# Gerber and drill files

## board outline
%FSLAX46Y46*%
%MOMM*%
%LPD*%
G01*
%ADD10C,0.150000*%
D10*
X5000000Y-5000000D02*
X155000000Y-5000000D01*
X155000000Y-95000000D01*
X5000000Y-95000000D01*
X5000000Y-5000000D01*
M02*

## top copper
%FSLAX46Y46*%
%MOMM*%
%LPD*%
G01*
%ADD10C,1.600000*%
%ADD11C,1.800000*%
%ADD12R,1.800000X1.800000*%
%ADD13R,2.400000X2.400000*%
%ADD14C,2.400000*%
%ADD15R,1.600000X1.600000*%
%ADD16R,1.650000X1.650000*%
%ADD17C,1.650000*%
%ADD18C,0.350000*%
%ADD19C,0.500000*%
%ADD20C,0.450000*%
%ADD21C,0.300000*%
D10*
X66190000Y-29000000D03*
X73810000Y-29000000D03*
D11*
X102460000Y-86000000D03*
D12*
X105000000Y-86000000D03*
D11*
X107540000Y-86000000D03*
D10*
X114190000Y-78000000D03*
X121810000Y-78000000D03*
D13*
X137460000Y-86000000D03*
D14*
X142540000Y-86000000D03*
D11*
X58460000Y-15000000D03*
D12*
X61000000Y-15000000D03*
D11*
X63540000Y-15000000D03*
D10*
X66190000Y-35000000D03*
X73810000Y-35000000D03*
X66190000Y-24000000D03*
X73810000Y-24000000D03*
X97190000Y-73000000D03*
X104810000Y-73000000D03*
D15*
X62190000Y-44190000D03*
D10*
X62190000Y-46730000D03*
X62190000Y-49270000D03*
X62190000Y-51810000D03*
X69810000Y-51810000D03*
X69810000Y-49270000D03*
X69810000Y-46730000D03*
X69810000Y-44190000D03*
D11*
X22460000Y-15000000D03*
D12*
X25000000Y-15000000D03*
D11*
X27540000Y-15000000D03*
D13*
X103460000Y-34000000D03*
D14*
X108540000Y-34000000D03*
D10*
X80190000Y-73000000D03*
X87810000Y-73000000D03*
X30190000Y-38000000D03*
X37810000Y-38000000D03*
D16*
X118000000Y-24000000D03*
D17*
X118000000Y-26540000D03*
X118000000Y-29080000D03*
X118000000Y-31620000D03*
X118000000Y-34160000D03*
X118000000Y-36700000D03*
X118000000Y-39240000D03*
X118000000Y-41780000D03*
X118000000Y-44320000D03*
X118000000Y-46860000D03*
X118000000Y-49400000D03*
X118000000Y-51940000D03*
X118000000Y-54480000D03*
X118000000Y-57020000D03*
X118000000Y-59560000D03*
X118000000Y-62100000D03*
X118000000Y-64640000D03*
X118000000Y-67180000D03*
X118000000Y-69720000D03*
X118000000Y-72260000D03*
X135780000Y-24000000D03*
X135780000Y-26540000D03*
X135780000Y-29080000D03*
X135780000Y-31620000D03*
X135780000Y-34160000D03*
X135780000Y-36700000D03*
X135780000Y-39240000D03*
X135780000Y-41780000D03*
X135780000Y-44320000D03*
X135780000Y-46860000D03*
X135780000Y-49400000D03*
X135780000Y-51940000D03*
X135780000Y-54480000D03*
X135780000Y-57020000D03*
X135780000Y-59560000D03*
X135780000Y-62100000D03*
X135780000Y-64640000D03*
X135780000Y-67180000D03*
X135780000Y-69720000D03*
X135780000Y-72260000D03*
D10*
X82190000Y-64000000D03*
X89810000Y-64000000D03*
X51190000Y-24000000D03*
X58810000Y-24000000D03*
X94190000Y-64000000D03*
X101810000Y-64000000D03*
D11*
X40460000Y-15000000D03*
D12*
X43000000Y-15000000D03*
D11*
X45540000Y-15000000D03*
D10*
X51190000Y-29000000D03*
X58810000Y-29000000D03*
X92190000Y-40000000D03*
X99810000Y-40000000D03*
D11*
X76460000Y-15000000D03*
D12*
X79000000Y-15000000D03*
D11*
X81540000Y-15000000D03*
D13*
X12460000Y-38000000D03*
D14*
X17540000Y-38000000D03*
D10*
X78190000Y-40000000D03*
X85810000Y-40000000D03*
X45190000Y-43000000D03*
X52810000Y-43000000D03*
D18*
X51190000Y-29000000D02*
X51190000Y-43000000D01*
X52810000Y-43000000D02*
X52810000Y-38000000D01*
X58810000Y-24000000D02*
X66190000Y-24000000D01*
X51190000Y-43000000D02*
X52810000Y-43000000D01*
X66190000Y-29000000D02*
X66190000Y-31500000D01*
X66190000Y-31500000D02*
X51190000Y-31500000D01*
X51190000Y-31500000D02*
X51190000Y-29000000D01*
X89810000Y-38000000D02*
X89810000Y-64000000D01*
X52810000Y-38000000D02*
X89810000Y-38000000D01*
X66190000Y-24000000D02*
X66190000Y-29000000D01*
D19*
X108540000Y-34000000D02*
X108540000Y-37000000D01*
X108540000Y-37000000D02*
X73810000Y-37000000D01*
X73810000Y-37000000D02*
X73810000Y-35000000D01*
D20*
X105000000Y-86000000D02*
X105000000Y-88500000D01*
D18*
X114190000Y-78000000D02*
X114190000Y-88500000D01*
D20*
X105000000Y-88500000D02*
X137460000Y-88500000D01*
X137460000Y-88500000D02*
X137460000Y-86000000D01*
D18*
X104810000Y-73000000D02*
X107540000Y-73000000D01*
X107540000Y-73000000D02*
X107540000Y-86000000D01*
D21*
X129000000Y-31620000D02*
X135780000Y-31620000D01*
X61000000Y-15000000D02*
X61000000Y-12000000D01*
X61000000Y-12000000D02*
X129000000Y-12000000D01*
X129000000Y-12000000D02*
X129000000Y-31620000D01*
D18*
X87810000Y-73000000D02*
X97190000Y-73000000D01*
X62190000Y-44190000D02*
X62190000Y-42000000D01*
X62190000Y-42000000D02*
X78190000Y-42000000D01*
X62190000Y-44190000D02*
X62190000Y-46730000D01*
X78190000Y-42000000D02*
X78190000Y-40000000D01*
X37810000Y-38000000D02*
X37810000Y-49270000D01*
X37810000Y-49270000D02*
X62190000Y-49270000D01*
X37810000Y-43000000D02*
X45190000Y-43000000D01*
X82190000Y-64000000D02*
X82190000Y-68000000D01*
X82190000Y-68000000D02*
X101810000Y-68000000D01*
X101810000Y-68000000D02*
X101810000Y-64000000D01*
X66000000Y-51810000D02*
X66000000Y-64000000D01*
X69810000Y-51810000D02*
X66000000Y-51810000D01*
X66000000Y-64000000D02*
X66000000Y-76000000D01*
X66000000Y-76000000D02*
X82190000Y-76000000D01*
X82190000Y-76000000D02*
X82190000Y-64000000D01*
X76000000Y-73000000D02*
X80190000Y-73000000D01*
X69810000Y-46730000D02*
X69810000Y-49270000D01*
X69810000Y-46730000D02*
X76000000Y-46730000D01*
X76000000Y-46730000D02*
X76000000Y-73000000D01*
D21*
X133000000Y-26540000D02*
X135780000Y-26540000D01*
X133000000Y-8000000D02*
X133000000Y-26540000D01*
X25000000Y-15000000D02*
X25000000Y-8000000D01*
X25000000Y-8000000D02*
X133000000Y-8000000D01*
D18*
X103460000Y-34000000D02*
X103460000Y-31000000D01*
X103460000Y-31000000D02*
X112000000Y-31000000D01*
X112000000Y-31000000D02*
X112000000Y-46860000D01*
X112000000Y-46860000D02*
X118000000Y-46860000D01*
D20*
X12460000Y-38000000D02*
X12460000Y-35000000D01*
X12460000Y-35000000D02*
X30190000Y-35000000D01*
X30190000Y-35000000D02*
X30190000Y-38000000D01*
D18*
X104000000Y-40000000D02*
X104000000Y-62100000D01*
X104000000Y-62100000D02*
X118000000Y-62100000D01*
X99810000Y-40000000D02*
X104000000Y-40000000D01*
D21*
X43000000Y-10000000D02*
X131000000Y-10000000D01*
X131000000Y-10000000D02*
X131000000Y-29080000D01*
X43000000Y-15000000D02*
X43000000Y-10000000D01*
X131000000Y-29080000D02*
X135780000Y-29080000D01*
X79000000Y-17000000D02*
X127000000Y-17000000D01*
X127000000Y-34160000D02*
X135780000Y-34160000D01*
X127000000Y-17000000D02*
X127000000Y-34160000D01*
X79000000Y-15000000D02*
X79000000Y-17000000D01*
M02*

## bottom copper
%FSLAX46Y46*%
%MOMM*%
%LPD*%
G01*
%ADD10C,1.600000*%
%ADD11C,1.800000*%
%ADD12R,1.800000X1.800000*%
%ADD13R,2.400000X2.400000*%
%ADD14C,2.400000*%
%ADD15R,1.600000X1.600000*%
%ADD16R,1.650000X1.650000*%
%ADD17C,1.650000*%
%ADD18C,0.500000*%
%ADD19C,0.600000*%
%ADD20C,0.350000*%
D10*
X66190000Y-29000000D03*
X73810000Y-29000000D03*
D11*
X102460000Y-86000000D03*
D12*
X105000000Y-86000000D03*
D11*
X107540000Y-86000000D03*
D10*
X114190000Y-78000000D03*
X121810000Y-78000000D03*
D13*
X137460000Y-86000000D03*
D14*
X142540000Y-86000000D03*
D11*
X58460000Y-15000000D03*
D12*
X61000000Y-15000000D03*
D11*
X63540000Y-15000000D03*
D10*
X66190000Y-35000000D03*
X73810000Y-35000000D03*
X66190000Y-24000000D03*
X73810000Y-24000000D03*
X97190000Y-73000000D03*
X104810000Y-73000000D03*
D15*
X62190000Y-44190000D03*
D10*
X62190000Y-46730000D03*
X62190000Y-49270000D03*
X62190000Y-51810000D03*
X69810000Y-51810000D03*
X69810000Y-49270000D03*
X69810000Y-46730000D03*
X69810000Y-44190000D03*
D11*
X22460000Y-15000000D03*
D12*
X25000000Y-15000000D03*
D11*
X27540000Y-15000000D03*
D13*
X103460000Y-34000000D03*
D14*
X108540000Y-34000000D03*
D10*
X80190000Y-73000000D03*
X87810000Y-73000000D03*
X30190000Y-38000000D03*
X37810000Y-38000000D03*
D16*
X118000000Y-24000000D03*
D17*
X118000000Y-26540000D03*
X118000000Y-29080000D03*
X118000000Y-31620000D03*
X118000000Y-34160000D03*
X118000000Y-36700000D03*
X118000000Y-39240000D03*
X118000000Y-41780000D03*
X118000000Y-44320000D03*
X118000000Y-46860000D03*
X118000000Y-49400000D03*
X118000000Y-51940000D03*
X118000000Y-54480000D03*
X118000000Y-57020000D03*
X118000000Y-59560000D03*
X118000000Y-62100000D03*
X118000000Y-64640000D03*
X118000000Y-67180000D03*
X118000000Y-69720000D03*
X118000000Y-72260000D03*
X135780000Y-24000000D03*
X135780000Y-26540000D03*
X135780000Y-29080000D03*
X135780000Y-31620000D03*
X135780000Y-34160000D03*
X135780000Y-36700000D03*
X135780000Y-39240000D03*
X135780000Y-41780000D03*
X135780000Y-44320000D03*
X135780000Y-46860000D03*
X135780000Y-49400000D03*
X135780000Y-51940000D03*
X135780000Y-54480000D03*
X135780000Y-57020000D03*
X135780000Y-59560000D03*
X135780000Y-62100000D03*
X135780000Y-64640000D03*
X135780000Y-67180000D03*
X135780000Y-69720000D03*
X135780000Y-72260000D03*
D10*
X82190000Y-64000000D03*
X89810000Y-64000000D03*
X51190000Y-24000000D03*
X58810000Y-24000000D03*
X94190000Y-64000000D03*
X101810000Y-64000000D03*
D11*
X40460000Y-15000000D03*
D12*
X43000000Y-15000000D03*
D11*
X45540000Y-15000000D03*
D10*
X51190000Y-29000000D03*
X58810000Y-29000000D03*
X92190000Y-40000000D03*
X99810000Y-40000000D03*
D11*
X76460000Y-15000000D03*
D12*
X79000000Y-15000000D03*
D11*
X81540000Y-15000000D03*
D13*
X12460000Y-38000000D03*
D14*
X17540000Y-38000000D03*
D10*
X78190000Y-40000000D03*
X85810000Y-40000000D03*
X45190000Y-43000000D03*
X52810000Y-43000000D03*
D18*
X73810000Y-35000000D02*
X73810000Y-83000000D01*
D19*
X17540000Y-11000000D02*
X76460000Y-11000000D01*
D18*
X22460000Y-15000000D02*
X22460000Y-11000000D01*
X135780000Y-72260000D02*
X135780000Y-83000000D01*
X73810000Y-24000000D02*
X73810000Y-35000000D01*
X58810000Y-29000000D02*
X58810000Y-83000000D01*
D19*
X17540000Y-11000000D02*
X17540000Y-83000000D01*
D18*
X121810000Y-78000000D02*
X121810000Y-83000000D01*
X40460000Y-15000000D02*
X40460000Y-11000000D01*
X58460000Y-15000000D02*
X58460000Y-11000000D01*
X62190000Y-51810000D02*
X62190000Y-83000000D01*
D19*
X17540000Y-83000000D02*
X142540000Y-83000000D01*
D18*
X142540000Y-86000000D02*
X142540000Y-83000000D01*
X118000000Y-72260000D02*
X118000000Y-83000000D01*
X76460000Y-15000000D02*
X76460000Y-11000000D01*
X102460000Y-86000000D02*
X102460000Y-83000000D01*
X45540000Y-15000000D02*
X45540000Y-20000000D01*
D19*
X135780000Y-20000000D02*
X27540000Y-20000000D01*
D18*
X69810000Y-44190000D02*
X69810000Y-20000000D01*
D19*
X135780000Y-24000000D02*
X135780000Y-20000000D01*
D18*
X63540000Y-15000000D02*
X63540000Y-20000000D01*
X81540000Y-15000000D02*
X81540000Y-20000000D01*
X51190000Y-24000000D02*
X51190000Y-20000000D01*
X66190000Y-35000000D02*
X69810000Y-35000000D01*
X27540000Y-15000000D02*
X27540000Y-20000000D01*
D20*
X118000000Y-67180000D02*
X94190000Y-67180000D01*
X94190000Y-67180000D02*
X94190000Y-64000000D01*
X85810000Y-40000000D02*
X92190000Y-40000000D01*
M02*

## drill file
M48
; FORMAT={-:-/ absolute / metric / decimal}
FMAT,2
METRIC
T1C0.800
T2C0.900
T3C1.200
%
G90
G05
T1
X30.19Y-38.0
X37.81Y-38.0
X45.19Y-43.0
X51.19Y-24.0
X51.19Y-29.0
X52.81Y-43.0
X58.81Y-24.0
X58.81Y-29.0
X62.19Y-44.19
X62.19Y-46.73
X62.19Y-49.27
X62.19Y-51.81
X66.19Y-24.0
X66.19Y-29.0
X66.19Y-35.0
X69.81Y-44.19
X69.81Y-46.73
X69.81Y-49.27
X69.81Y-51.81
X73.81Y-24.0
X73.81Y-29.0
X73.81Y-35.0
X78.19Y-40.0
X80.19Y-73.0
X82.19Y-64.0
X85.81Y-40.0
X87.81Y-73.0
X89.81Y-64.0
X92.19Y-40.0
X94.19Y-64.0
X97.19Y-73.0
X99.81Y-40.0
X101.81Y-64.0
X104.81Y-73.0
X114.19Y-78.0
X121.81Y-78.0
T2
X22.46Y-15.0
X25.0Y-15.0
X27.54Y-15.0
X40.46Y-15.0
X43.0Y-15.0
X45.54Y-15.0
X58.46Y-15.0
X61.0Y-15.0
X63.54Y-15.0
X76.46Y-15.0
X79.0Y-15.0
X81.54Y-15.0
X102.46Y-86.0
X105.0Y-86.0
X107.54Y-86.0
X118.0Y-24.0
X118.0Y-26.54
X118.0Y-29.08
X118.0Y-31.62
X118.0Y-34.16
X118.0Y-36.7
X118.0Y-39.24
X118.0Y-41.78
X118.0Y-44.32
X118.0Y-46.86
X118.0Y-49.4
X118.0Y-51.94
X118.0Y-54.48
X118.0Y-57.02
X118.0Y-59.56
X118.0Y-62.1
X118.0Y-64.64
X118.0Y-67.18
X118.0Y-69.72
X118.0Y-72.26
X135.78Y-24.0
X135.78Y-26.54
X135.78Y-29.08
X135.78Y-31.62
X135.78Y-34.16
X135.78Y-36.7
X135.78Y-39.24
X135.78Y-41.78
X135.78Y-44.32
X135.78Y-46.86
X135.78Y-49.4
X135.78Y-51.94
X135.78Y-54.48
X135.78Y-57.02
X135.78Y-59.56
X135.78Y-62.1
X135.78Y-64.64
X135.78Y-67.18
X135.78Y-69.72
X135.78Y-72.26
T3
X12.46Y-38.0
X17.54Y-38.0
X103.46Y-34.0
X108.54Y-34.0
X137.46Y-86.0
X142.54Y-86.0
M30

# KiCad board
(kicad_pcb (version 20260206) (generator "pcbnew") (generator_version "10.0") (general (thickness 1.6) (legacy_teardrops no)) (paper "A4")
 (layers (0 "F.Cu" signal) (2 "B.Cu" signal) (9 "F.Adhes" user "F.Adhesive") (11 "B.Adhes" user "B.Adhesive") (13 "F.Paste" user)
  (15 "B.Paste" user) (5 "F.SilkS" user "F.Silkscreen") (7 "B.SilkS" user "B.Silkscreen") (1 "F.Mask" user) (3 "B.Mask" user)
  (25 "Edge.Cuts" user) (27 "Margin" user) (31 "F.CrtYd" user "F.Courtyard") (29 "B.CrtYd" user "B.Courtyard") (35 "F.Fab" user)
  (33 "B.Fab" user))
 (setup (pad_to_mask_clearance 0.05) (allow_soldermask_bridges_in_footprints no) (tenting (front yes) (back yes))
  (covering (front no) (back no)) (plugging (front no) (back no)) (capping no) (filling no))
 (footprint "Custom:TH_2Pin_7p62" (layer "F.Cu") (at 70 29)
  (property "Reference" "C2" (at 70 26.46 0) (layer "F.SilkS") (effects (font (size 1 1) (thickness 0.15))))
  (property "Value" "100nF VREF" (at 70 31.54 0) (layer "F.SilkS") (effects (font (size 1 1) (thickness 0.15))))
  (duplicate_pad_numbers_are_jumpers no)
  (pad "1" thru_hole circle (at -3.81 0) (size 1.6 1.6) (drill 0.8) (layers "*.Cu" "*.Mask") (remove_unused_layers no) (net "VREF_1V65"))
  (pad "2" thru_hole circle (at 3.81 0) (size 1.6 1.6) (drill 0.8) (layers "*.Cu" "*.Mask") (remove_unused_layers no) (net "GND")))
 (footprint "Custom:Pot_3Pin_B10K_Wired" (layer "F.Cu") (at 105 86)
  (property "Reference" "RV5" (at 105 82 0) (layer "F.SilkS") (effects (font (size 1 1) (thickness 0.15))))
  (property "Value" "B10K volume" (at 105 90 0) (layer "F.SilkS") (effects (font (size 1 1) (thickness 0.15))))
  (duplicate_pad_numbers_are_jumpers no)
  (pad "1" thru_hole circle (at -2.54 0) (size 1.8 1.8) (drill 0.9) (layers "*.Cu" "*.Mask") (remove_unused_layers no) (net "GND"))
  (pad "2" thru_hole rect (at 0 0) (size 1.8 1.8) (drill 0.9) (layers "*.Cu" "*.Mask") (remove_unused_layers no) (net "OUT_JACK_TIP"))
  (pad "3" thru_hole circle (at 2.54 0) (size 1.8 1.8) (drill 0.9) (layers "*.Cu" "*.Mask") (remove_unused_layers no) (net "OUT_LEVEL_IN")))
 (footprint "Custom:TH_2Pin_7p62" (layer "F.Cu") (at 118 78)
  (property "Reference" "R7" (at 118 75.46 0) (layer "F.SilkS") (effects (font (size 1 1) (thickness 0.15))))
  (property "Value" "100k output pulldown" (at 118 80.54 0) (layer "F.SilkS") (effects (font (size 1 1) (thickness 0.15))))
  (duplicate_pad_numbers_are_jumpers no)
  (pad "1" thru_hole circle (at -3.81 0) (size 1.6 1.6) (drill 0.8) (layers "*.Cu" "*.Mask") (remove_unused_layers no) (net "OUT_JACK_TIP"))
  (pad "2" thru_hole circle (at 3.81 0) (size 1.6 1.6) (drill 0.8) (layers "*.Cu" "*.Mask") (remove_unused_layers no) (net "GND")))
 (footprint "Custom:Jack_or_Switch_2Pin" (layer "F.Cu") (at 140 86)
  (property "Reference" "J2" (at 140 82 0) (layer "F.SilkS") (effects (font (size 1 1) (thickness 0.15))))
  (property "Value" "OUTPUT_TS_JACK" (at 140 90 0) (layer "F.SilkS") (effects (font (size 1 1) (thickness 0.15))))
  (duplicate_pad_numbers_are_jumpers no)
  (pad "1" thru_hole rect (at -2.54 0) (size 2.4 2.4) (drill 1.2) (layers "*.Cu" "*.Mask") (remove_unused_layers no) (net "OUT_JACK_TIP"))
  (pad "2" thru_hole circle (at 2.54 0) (size 2.4 2.4) (drill 1.2) (layers "*.Cu" "*.Mask") (remove_unused_layers no) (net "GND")))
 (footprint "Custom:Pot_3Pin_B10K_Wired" (layer "F.Cu") (at 61 15)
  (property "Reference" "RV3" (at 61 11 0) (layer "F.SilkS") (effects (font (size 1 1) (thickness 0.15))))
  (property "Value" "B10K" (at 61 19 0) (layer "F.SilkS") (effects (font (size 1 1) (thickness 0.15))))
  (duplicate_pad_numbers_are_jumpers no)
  (pad "1" thru_hole circle (at -2.54 0) (size 1.8 1.8) (drill 0.9) (layers "*.Cu" "*.Mask") (remove_unused_layers no) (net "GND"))
  (pad "2" thru_hole rect (at 0 0) (size 1.8 1.8) (drill 0.9) (layers "*.Cu" "*.Mask") (remove_unused_layers no) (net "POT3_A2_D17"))
  (pad "3" thru_hole circle (at 2.54 0) (size 1.8 1.8) (drill 0.9) (layers "*.Cu" "*.Mask") (remove_unused_layers no) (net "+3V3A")))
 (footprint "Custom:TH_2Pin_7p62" (layer "F.Cu") (at 70 35)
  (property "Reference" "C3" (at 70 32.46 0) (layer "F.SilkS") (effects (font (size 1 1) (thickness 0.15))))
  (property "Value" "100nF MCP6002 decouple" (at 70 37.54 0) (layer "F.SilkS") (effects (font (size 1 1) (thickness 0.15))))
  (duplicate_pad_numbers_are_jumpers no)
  (pad "1" thru_hole circle (at -3.81 0) (size 1.6 1.6) (drill 0.8) (layers "*.Cu" "*.Mask") (remove_unused_layers no) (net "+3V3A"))
  (pad "2" thru_hole circle (at 3.81 0) (size 1.6 1.6) (drill 0.8) (layers "*.Cu" "*.Mask") (remove_unused_layers no) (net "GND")))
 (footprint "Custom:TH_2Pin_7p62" (layer "F.Cu") (at 70 24)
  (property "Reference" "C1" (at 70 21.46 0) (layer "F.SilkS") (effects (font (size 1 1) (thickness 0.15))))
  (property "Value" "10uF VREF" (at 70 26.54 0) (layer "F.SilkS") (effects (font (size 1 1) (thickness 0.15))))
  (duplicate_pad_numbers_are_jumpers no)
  (pad "1" thru_hole circle (at -3.81 0) (size 1.6 1.6) (drill 0.8) (layers "*.Cu" "*.Mask") (remove_unused_layers no) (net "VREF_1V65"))
  (pad "2" thru_hole circle (at 3.81 0) (size 1.6 1.6) (drill 0.8) (layers "*.Cu" "*.Mask") (remove_unused_layers no) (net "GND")))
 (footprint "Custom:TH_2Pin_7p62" (layer "F.Cu") (at 101 73)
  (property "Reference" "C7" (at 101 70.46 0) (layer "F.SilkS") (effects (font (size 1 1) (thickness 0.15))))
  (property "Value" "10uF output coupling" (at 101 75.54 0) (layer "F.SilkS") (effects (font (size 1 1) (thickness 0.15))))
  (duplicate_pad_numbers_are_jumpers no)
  (pad "1" thru_hole circle (at -3.81 0) (size 1.6 1.6) (drill 0.8) (layers "*.Cu" "*.Mask") (remove_unused_layers no) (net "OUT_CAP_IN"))
  (pad "2" thru_hole circle (at 3.81 0) (size 1.6 1.6) (drill 0.8) (layers "*.Cu" "*.Mask") (remove_unused_layers no) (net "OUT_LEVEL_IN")))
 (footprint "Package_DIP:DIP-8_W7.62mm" (layer "F.Cu") (at 66 48)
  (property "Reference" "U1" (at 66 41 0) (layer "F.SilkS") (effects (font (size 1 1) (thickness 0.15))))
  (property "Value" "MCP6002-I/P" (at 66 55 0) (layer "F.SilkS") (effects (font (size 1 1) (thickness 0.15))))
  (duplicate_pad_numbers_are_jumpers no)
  (pad "1" thru_hole rect (at -3.81 -3.81) (size 1.6 1.6) (drill 0.8) (layers "*.Cu" "*.Mask") (remove_unused_layers no) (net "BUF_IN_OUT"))
  (pad "2" thru_hole circle (at -3.81 -1.27) (size 1.6 1.6) (drill 0.8) (layers "*.Cu" "*.Mask") (remove_unused_layers no)
   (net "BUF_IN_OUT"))
  (pad "3" thru_hole circle (at -3.81 1.27) (size 1.6 1.6) (drill 0.8) (layers "*.Cu" "*.Mask") (remove_unused_layers no) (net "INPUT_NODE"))
  (pad "4" thru_hole circle (at -3.81 3.81) (size 1.6 1.6) (drill 0.8) (layers "*.Cu" "*.Mask") (remove_unused_layers no) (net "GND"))
  (pad "5" thru_hole circle (at 3.81 3.81) (size 1.6 1.6) (drill 0.8) (layers "*.Cu" "*.Mask") (remove_unused_layers no)
   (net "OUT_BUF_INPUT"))
  (pad "6" thru_hole circle (at 3.81 1.27) (size 1.6 1.6) (drill 0.8) (layers "*.Cu" "*.Mask") (remove_unused_layers no) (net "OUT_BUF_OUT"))
  (pad "7" thru_hole circle (at 3.81 -1.27) (size 1.6 1.6) (drill 0.8) (layers "*.Cu" "*.Mask") (remove_unused_layers no)
   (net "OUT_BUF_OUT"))
  (pad "8" thru_hole circle (at 3.81 -3.81) (size 1.6 1.6) (drill 0.8) (layers "*.Cu" "*.Mask") (remove_unused_layers no) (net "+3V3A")))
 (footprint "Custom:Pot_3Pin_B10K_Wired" (layer "F.Cu") (at 25 15)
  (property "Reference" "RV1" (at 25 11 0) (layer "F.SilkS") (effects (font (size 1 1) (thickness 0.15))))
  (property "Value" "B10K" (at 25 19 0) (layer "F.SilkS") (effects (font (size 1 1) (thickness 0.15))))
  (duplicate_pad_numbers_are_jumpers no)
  (pad "1" thru_hole circle (at -2.54 0) (size 1.8 1.8) (drill 0.9) (layers "*.Cu" "*.Mask") (remove_unused_layers no) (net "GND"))
  (pad "2" thru_hole rect (at 0 0) (size 1.8 1.8) (drill 0.9) (layers "*.Cu" "*.Mask") (remove_unused_layers no) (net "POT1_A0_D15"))
  (pad "3" thru_hole circle (at 2.54 0) (size 1.8 1.8) (drill 0.9) (layers "*.Cu" "*.Mask") (remove_unused_layers no) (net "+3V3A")))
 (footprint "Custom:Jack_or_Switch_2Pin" (layer "F.Cu") (at 106 34)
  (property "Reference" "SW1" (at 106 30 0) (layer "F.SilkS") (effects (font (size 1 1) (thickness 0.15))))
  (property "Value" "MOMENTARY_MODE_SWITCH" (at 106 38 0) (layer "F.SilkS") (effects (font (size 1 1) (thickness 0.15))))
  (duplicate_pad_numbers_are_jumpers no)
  (pad "1" thru_hole rect (at -2.54 0) (size 2.4 2.4) (drill 1.2) (layers "*.Cu" "*.Mask") (remove_unused_layers no) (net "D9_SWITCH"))
  (pad "2" thru_hole circle (at 2.54 0) (size 2.4 2.4) (drill 1.2) (layers "*.Cu" "*.Mask") (remove_unused_layers no) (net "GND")))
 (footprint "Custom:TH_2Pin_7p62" (layer "F.Cu") (at 84 73)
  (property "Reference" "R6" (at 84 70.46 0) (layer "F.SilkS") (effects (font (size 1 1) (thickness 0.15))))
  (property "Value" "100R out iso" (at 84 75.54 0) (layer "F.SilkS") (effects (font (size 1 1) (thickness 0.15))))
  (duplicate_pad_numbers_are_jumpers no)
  (pad "1" thru_hole circle (at -3.81 0) (size 1.6 1.6) (drill 0.8) (layers "*.Cu" "*.Mask") (remove_unused_layers no) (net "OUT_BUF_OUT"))
  (pad "2" thru_hole circle (at 3.81 0) (size 1.6 1.6) (drill 0.8) (layers "*.Cu" "*.Mask") (remove_unused_layers no) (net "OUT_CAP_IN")))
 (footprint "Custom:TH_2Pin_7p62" (layer "F.Cu") (at 34 38)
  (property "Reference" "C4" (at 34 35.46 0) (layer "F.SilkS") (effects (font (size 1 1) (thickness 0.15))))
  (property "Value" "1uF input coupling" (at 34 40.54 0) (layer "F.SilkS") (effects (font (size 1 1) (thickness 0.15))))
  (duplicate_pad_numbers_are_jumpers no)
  (pad "1" thru_hole circle (at -3.81 0) (size 1.6 1.6) (drill 0.8) (layers "*.Cu" "*.Mask") (remove_unused_layers no) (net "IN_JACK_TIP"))
  (pad "2" thru_hole circle (at 3.81 0) (size 1.6 1.6) (drill 0.8) (layers "*.Cu" "*.Mask") (remove_unused_layers no) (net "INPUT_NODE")))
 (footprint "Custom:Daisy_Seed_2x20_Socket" (layer "F.Cu") (at 118 24)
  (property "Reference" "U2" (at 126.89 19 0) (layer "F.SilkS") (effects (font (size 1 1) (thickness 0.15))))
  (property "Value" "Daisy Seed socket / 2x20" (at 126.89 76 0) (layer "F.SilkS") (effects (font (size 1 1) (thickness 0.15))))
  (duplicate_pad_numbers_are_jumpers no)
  (pad "1" thru_hole rect (at 0 0) (size 1.65 1.65) (drill 0.9) (layers "*.Cu" "*.Mask") (remove_unused_layers no))
  (pad "2" thru_hole circle (at 0 2.54) (size 1.65 1.65) (drill 0.9) (layers "*.Cu" "*.Mask") (remove_unused_layers no))
  (pad "3" thru_hole circle (at 0 5.08) (size 1.65 1.65) (drill 0.9) (layers "*.Cu" "*.Mask") (remove_unused_layers no))
  (pad "4" thru_hole circle (at 0 7.62) (size 1.65 1.65) (drill 0.9) (layers "*.Cu" "*.Mask") (remove_unused_layers no))
  (pad "5" thru_hole circle (at 0 10.16) (size 1.65 1.65) (drill 0.9) (layers "*.Cu" "*.Mask") (remove_unused_layers no))
  (pad "6" thru_hole circle (at 0 12.7) (size 1.65 1.65) (drill 0.9) (layers "*.Cu" "*.Mask") (remove_unused_layers no))
  (pad "7" thru_hole circle (at 0 15.24) (size 1.65 1.65) (drill 0.9) (layers "*.Cu" "*.Mask") (remove_unused_layers no))
  (pad "8" thru_hole circle (at 0 17.78) (size 1.65 1.65) (drill 0.9) (layers "*.Cu" "*.Mask") (remove_unused_layers no))
  (pad "9" thru_hole circle (at 0 20.32) (size 1.65 1.65) (drill 0.9) (layers "*.Cu" "*.Mask") (remove_unused_layers no))
  (pad "10" thru_hole circle (at 0 22.86) (size 1.65 1.65) (drill 0.9) (layers "*.Cu" "*.Mask") (remove_unused_layers no) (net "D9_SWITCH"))
  (pad "11" thru_hole circle (at 0 25.4) (size 1.65 1.65) (drill 0.9) (layers "*.Cu" "*.Mask") (remove_unused_layers no))
  (pad "12" thru_hole circle (at 0 27.94) (size 1.65 1.65) (drill 0.9) (layers "*.Cu" "*.Mask") (remove_unused_layers no))
  (pad "13" thru_hole circle (at 0 30.48) (size 1.65 1.65) (drill 0.9) (layers "*.Cu" "*.Mask") (remove_unused_layers no))
  (pad "14" thru_hole circle (at 0 33.02) (size 1.65 1.65) (drill 0.9) (layers "*.Cu" "*.Mask") (remove_unused_layers no))
  (pad "15" thru_hole circle (at 0 35.56) (size 1.65 1.65) (drill 0.9) (layers "*.Cu" "*.Mask") (remove_unused_layers no))
  (pad "16" thru_hole circle (at 0 38.1) (size 1.65 1.65) (drill 0.9) (layers "*.Cu" "*.Mask") (remove_unused_layers no) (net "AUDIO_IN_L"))
  (pad "17" thru_hole circle (at 0 40.64) (size 1.65 1.65) (drill 0.9) (layers "*.Cu" "*.Mask") (remove_unused_layers no))
  (pad "18" thru_hole circle (at 0 43.18) (size 1.65 1.65) (drill 0.9) (layers "*.Cu" "*.Mask") (remove_unused_layers no)
   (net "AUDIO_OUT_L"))
  (pad "19" thru_hole circle (at 0 45.72) (size 1.65 1.65) (drill 0.9) (layers "*.Cu" "*.Mask") (remove_unused_layers no)
   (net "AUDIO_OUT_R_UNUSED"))
  (pad "20" thru_hole circle (at 0 48.26) (size 1.65 1.65) (drill 0.9) (layers "*.Cu" "*.Mask") (remove_unused_layers no) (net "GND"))
  (pad "21" thru_hole circle (at 17.78 0) (size 1.65 1.65) (drill 0.9) (layers "*.Cu" "*.Mask") (remove_unused_layers no) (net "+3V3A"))
  (pad "22" thru_hole circle (at 17.78 2.54) (size 1.65 1.65) (drill 0.9) (layers "*.Cu" "*.Mask") (remove_unused_layers no)
   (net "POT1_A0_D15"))
  (pad "23" thru_hole circle (at 17.78 5.08) (size 1.65 1.65) (drill 0.9) (layers "*.Cu" "*.Mask") (remove_unused_layers no)
   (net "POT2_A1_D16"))
  (pad "24" thru_hole circle (at 17.78 7.62) (size 1.65 1.65) (drill 0.9) (layers "*.Cu" "*.Mask") (remove_unused_layers no)
   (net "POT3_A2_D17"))
  (pad "25" thru_hole circle (at 17.78 10.16) (size 1.65 1.65) (drill 0.9) (layers "*.Cu" "*.Mask") (remove_unused_layers no)
   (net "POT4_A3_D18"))
  (pad "26" thru_hole circle (at 17.78 12.7) (size 1.65 1.65) (drill 0.9) (layers "*.Cu" "*.Mask") (remove_unused_layers no))
  (pad "27" thru_hole circle (at 17.78 15.24) (size 1.65 1.65) (drill 0.9) (layers "*.Cu" "*.Mask") (remove_unused_layers no))
  (pad "28" thru_hole circle (at 17.78 17.78) (size 1.65 1.65) (drill 0.9) (layers "*.Cu" "*.Mask") (remove_unused_layers no))
  (pad "29" thru_hole circle (at 17.78 20.32) (size 1.65 1.65) (drill 0.9) (layers "*.Cu" "*.Mask") (remove_unused_layers no))
  (pad "30" thru_hole circle (at 17.78 22.86) (size 1.65 1.65) (drill 0.9) (layers "*.Cu" "*.Mask") (remove_unused_layers no))
  (pad "31" thru_hole circle (at 17.78 25.4) (size 1.65 1.65) (drill 0.9) (layers "*.Cu" "*.Mask") (remove_unused_layers no))
  (pad "32" thru_hole circle (at 17.78 27.94) (size 1.65 1.65) (drill 0.9) (layers "*.Cu" "*.Mask") (remove_unused_layers no))
  (pad "33" thru_hole circle (at 17.78 30.48) (size 1.65 1.65) (drill 0.9) (layers "*.Cu" "*.Mask") (remove_unused_layers no))
  (pad "34" thru_hole circle (at 17.78 33.02) (size 1.65 1.65) (drill 0.9) (layers "*.Cu" "*.Mask") (remove_unused_layers no))
  (pad "35" thru_hole circle (at 17.78 35.56) (size 1.65 1.65) (drill 0.9) (layers "*.Cu" "*.Mask") (remove_unused_layers no))
  (pad "36" thru_hole circle (at 17.78 38.1) (size 1.65 1.65) (drill 0.9) (layers "*.Cu" "*.Mask") (remove_unused_layers no))
  (pad "37" thru_hole circle (at 17.78 40.64) (size 1.65 1.65) (drill 0.9) (layers "*.Cu" "*.Mask") (remove_unused_layers no))
  (pad "38" thru_hole circle (at 17.78 43.18) (size 1.65 1.65) (drill 0.9) (layers "*.Cu" "*.Mask") (remove_unused_layers no))
  (pad "39" thru_hole circle (at 17.78 45.72) (size 1.65 1.65) (drill 0.9) (layers "*.Cu" "*.Mask") (remove_unused_layers no))
  (pad "40" thru_hole circle (at 17.78 48.26) (size 1.65 1.65) (drill 0.9) (layers "*.Cu" "*.Mask") (remove_unused_layers no) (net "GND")))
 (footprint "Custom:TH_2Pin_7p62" (layer "F.Cu") (at 86 64)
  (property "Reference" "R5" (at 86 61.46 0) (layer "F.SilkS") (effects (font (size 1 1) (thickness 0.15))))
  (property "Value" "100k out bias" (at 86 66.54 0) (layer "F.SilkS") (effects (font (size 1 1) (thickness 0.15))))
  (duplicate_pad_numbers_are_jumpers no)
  (pad "1" thru_hole circle (at -3.81 0) (size 1.6 1.6) (drill 0.8) (layers "*.Cu" "*.Mask") (remove_unused_layers no) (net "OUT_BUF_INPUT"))
  (pad "2" thru_hole circle (at 3.81 0) (size 1.6 1.6) (drill 0.8) (layers "*.Cu" "*.Mask") (remove_unused_layers no) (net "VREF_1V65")))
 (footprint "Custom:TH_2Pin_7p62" (layer "F.Cu") (at 55 24)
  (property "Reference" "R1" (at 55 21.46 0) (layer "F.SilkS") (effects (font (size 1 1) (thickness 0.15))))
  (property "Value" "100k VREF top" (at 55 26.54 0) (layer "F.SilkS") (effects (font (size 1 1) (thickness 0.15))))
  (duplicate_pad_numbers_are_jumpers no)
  (pad "1" thru_hole circle (at -3.81 0) (size 1.6 1.6) (drill 0.8) (layers "*.Cu" "*.Mask") (remove_unused_layers no) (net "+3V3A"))
  (pad "2" thru_hole circle (at 3.81 0) (size 1.6 1.6) (drill 0.8) (layers "*.Cu" "*.Mask") (remove_unused_layers no) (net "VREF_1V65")))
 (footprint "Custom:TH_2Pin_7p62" (layer "F.Cu") (at 98 64)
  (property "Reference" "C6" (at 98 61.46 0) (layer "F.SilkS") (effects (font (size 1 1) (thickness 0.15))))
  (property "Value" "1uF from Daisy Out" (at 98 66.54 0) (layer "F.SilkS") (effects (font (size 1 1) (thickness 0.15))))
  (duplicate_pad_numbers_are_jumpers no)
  (pad "1" thru_hole circle (at -3.81 0) (size 1.6 1.6) (drill 0.8) (layers "*.Cu" "*.Mask") (remove_unused_layers no) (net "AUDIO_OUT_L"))
  (pad "2" thru_hole circle (at 3.81 0) (size 1.6 1.6) (drill 0.8) (layers "*.Cu" "*.Mask") (remove_unused_layers no) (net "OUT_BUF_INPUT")))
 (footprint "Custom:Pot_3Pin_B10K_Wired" (layer "F.Cu") (at 43 15)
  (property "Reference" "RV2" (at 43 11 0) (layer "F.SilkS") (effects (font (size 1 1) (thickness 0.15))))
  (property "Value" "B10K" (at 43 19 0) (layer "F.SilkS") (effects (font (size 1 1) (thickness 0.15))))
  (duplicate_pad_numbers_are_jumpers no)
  (pad "1" thru_hole circle (at -2.54 0) (size 1.8 1.8) (drill 0.9) (layers "*.Cu" "*.Mask") (remove_unused_layers no) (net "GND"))
  (pad "2" thru_hole rect (at 0 0) (size 1.8 1.8) (drill 0.9) (layers "*.Cu" "*.Mask") (remove_unused_layers no) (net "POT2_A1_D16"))
  (pad "3" thru_hole circle (at 2.54 0) (size 1.8 1.8) (drill 0.9) (layers "*.Cu" "*.Mask") (remove_unused_layers no) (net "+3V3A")))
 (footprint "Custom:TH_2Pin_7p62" (layer "F.Cu") (at 55 29)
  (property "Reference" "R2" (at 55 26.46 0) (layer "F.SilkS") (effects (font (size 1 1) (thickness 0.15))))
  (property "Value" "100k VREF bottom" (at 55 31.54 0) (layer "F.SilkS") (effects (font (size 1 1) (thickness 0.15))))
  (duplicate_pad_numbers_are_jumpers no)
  (pad "1" thru_hole circle (at -3.81 0) (size 1.6 1.6) (drill 0.8) (layers "*.Cu" "*.Mask") (remove_unused_layers no) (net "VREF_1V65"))
  (pad "2" thru_hole circle (at 3.81 0) (size 1.6 1.6) (drill 0.8) (layers "*.Cu" "*.Mask") (remove_unused_layers no) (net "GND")))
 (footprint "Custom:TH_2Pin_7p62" (layer "F.Cu") (at 96 40)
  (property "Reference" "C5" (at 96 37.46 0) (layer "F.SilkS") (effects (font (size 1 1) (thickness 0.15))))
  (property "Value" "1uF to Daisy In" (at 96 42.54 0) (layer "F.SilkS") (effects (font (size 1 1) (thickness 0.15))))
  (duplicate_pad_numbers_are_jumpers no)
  (pad "1" thru_hole circle (at -3.81 0) (size 1.6 1.6) (drill 0.8) (layers "*.Cu" "*.Mask") (remove_unused_layers no)
   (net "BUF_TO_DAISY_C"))
  (pad "2" thru_hole circle (at 3.81 0) (size 1.6 1.6) (drill 0.8) (layers "*.Cu" "*.Mask") (remove_unused_layers no) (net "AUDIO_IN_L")))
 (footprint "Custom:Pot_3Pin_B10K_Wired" (layer "F.Cu") (at 79 15)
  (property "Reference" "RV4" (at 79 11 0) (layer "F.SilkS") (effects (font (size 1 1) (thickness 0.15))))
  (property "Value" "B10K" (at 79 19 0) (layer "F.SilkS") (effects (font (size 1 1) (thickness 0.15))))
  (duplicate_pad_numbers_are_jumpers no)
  (pad "1" thru_hole circle (at -2.54 0) (size 1.8 1.8) (drill 0.9) (layers "*.Cu" "*.Mask") (remove_unused_layers no) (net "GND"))
  (pad "2" thru_hole rect (at 0 0) (size 1.8 1.8) (drill 0.9) (layers "*.Cu" "*.Mask") (remove_unused_layers no) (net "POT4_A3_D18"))
  (pad "3" thru_hole circle (at 2.54 0) (size 1.8 1.8) (drill 0.9) (layers "*.Cu" "*.Mask") (remove_unused_layers no) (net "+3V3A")))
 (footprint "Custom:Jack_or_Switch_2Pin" (layer "F.Cu") (at 15 38)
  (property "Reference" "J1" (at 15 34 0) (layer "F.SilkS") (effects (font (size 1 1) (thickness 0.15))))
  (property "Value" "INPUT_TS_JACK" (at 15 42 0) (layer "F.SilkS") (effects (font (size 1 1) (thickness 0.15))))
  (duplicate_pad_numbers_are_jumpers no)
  (pad "1" thru_hole rect (at -2.54 0) (size 2.4 2.4) (drill 1.2) (layers "*.Cu" "*.Mask") (remove_unused_layers no) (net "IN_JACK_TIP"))
  (pad "2" thru_hole circle (at 2.54 0) (size 2.4 2.4) (drill 1.2) (layers "*.Cu" "*.Mask") (remove_unused_layers no) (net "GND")))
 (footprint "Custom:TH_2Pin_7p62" (layer "F.Cu") (at 82 40)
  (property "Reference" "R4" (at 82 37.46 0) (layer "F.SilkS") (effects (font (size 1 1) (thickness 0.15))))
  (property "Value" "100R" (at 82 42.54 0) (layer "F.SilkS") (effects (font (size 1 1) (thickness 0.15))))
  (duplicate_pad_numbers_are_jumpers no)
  (pad "1" thru_hole circle (at -3.81 0) (size 1.6 1.6) (drill 0.8) (layers "*.Cu" "*.Mask") (remove_unused_layers no) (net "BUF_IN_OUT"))
  (pad "2" thru_hole circle (at 3.81 0) (size 1.6 1.6) (drill 0.8) (layers "*.Cu" "*.Mask") (remove_unused_layers no) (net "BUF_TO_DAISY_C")))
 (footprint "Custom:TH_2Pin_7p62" (layer "F.Cu") (at 49 43)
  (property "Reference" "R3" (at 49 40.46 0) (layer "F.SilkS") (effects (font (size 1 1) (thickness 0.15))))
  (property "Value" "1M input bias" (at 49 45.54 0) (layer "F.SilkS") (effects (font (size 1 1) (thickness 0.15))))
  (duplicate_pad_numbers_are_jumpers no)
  (pad "1" thru_hole circle (at -3.81 0) (size 1.6 1.6) (drill 0.8) (layers "*.Cu" "*.Mask") (remove_unused_layers no) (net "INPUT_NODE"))
  (pad "2" thru_hole circle (at 3.81 0) (size 1.6 1.6) (drill 0.8) (layers "*.Cu" "*.Mask") (remove_unused_layers no) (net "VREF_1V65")))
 (gr_rect (start 5 5) (end 155 95) (stroke (width 0.15) (type solid)) (fill no) (layer "Edge.Cuts"))
 (segment (start 51.19 29) (end 51.19 43) (width 0.35) (layer "F.Cu") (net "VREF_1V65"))
 (segment (start 52.81 43) (end 52.81 38) (width 0.35) (layer "F.Cu") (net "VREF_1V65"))
 (segment (start 58.81 24) (end 66.19 24) (width 0.35) (layer "F.Cu") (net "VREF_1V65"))
 (segment (start 51.19 43) (end 52.81 43) (width 0.35) (layer "F.Cu") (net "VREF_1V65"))
 (segment (start 66.19 29) (end 66.19 31.5) (width 0.35) (layer "F.Cu") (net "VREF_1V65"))
 (segment (start 66.19 31.5) (end 51.19 31.5) (width 0.35) (layer "F.Cu") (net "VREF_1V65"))
 (segment (start 51.19 31.5) (end 51.19 29) (width 0.35) (layer "F.Cu") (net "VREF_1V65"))
 (segment (start 89.81 38) (end 89.81 64) (width 0.35) (layer "F.Cu") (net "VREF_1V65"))
 (segment (start 52.81 38) (end 89.81 38) (width 0.35) (layer "F.Cu") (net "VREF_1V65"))
 (segment (start 66.19 24) (end 66.19 29) (width 0.35) (layer "F.Cu") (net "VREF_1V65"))
 (segment (start 108.54 34) (end 108.54 37) (width 0.5) (layer "F.Cu") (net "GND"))
 (segment (start 108.54 37) (end 73.81 37) (width 0.5) (layer "F.Cu") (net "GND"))
 (segment (start 73.81 37) (end 73.81 35) (width 0.5) (layer "F.Cu") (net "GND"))
 (segment (start 73.81 35) (end 73.81 83) (width 0.5) (layer "B.Cu") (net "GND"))
 (segment (start 17.54 11) (end 76.46 11) (width 0.6) (layer "B.Cu") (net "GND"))
 (segment (start 22.46 15) (end 22.46 11) (width 0.5) (layer "B.Cu") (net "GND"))
 (segment (start 135.78 72.26) (end 135.78 83) (width 0.5) (layer "B.Cu") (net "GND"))
 (segment (start 73.81 24) (end 73.81 35) (width 0.5) (layer "B.Cu") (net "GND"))
 (segment (start 58.81 29) (end 58.81 83) (width 0.5) (layer "B.Cu") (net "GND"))
 (segment (start 17.54 11) (end 17.54 83) (width 0.6) (layer "B.Cu") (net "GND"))
 (segment (start 121.81 78) (end 121.81 83) (width 0.5) (layer "B.Cu") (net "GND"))
 (segment (start 40.46 15) (end 40.46 11) (width 0.5) (layer "B.Cu") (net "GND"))
 (segment (start 58.46 15) (end 58.46 11) (width 0.5) (layer "B.Cu") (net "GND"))
 (segment (start 62.19 51.81) (end 62.19 83) (width 0.5) (layer "B.Cu") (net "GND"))
 (segment (start 17.54 83) (end 142.54 83) (width 0.6) (layer "B.Cu") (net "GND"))
 (segment (start 142.54 86) (end 142.54 83) (width 0.5) (layer "B.Cu") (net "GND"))
 (segment (start 118 72.26) (end 118 83) (width 0.5) (layer "B.Cu") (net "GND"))
 (segment (start 76.46 15) (end 76.46 11) (width 0.5) (layer "B.Cu") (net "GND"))
 (segment (start 102.46 86) (end 102.46 83) (width 0.5) (layer "B.Cu") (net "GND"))
 (segment (start 105 86) (end 105 88.5) (width 0.45) (layer "F.Cu") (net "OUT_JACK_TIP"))
 (segment (start 114.19 78) (end 114.19 88.5) (width 0.35) (layer "F.Cu") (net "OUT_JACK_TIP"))
 (segment (start 105 88.5) (end 137.46 88.5) (width 0.45) (layer "F.Cu") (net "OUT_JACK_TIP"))
 (segment (start 137.46 88.5) (end 137.46 86) (width 0.45) (layer "F.Cu") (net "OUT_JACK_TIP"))
 (segment (start 104.81 73) (end 107.54 73) (width 0.35) (layer "F.Cu") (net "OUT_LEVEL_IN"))
 (segment (start 107.54 73) (end 107.54 86) (width 0.35) (layer "F.Cu") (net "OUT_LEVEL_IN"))
 (segment (start 129 31.62) (end 135.78 31.62) (width 0.3) (layer "F.Cu") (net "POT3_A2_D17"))
 (segment (start 61 15) (end 61 12) (width 0.3) (layer "F.Cu") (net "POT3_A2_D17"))
 (segment (start 61 12) (end 129 12) (width 0.3) (layer "F.Cu") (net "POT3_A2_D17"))
 (segment (start 129 12) (end 129 31.62) (width 0.3) (layer "F.Cu") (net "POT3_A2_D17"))
 (segment (start 45.54 15) (end 45.54 20) (width 0.5) (layer "B.Cu") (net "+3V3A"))
 (segment (start 135.78 20) (end 27.54 20) (width 0.6) (layer "B.Cu") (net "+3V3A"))
 (segment (start 69.81 44.19) (end 69.81 20) (width 0.5) (layer "B.Cu") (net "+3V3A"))
 (segment (start 135.78 24) (end 135.78 20) (width 0.6) (layer "B.Cu") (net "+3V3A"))
 (segment (start 63.54 15) (end 63.54 20) (width 0.5) (layer "B.Cu") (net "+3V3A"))
 (segment (start 81.54 15) (end 81.54 20) (width 0.5) (layer "B.Cu") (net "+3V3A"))
 (segment (start 51.19 24) (end 51.19 20) (width 0.5) (layer "B.Cu") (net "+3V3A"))
 (segment (start 66.19 35) (end 69.81 35) (width 0.5) (layer "B.Cu") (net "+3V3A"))
 (segment (start 27.54 15) (end 27.54 20) (width 0.5) (layer "B.Cu") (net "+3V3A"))
 (segment (start 87.81 73) (end 97.19 73) (width 0.35) (layer "F.Cu") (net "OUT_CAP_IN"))
 (segment (start 62.19 44.19) (end 62.19 42) (width 0.35) (layer "F.Cu") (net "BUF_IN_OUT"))
 (segment (start 62.19 42) (end 78.19 42) (width 0.35) (layer "F.Cu") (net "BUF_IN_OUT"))
 (segment (start 62.19 44.19) (end 62.19 46.73) (width 0.35) (layer "F.Cu") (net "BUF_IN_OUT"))
 (segment (start 78.19 42) (end 78.19 40) (width 0.35) (layer "F.Cu") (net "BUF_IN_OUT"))
 (segment (start 37.81 38) (end 37.81 49.27) (width 0.35) (layer "F.Cu") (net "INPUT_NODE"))
 (segment (start 37.81 49.27) (end 62.19 49.27) (width 0.35) (layer "F.Cu") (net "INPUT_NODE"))
 (segment (start 37.81 43) (end 45.19 43) (width 0.35) (layer "F.Cu") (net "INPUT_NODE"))
 (segment (start 82.19 64) (end 82.19 68) (width 0.35) (layer "F.Cu") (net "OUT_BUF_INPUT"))
 (segment (start 82.19 68) (end 101.81 68) (width 0.35) (layer "F.Cu") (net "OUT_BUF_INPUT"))
 (segment (start 101.81 68) (end 101.81 64) (width 0.35) (layer "F.Cu") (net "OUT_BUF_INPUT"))
 (segment (start 66 51.81) (end 66 64) (width 0.35) (layer "F.Cu") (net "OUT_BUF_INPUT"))
 (segment (start 69.81 51.81) (end 66 51.81) (width 0.35) (layer "F.Cu") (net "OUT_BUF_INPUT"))
 (segment (start 66 64) (end 66 76) (width 0.35) (layer "F.Cu") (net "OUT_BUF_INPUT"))
 (segment (start 66 76) (end 82.19 76) (width 0.35) (layer "F.Cu") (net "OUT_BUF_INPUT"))
 (segment (start 82.19 76) (end 82.19 64) (width 0.35) (layer "F.Cu") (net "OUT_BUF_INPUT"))
 (segment (start 76 73) (end 80.19 73) (width 0.35) (layer "F.Cu") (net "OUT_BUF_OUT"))
 (segment (start 69.81 46.73) (end 69.81 49.27) (width 0.35) (layer "F.Cu") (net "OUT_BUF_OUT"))
 (segment (start 69.81 46.73) (end 76 46.73) (width 0.35) (layer "F.Cu") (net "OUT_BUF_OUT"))
 (segment (start 76 46.73) (end 76 73) (width 0.35) (layer "F.Cu") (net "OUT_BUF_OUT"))
 (segment (start 133 26.54) (end 135.78 26.54) (width 0.3) (layer "F.Cu") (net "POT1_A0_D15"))
 (segment (start 133 8) (end 133 26.54) (width 0.3) (layer "F.Cu") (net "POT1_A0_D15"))
 (segment (start 25 15) (end 25 8) (width 0.3) (layer "F.Cu") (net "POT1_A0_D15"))
 (segment (start 25 8) (end 133 8) (width 0.3) (layer "F.Cu") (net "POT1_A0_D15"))
 (segment (start 103.46 34) (end 103.46 31) (width 0.35) (layer "F.Cu") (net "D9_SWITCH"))
 (segment (start 103.46 31) (end 112 31) (width 0.35) (layer "F.Cu") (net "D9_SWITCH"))
 (segment (start 112 31) (end 112 46.86) (width 0.35) (layer "F.Cu") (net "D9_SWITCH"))
 (segment (start 112 46.86) (end 118 46.86) (width 0.35) (layer "F.Cu") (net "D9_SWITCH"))
 (segment (start 12.46 38) (end 12.46 35) (width 0.45) (layer "F.Cu") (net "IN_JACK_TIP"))
 (segment (start 12.46 35) (end 30.19 35) (width 0.45) (layer "F.Cu") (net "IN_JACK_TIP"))
 (segment (start 30.19 35) (end 30.19 38) (width 0.45) (layer "F.Cu") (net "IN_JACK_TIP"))
 (segment (start 104 40) (end 104 62.1) (width 0.35) (layer "F.Cu") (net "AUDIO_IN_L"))
 (segment (start 104 62.1) (end 118 62.1) (width 0.35) (layer "F.Cu") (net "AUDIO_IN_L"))
 (segment (start 99.81 40) (end 104 40) (width 0.35) (layer "F.Cu") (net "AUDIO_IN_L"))
 (segment (start 118 67.18) (end 94.19 67.18) (width 0.35) (layer "B.Cu") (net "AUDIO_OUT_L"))
 (segment (start 94.19 67.18) (end 94.19 64) (width 0.35) (layer "B.Cu") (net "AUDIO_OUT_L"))
 (segment (start 43 10) (end 131 10) (width 0.3) (layer "F.Cu") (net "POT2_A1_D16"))
 (segment (start 131 10) (end 131 29.08) (width 0.3) (layer "F.Cu") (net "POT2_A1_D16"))
 (segment (start 43 15) (end 43 10) (width 0.3) (layer "F.Cu") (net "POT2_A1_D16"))
 (segment (start 131 29.08) (end 135.78 29.08) (width 0.3) (layer "F.Cu") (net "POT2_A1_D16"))
 (segment (start 79 17) (end 127 17) (width 0.3) (layer "F.Cu") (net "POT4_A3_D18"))
 (segment (start 127 34.16) (end 135.78 34.16) (width 0.3) (layer "F.Cu") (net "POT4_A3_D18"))
 (segment (start 127 17) (end 127 34.16) (width 0.3) (layer "F.Cu") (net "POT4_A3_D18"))
 (segment (start 79 15) (end 79 17) (width 0.3) (layer "F.Cu") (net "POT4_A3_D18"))
 (segment (start 85.81 40) (end 92.19 40) (width 0.35) (layer "B.Cu") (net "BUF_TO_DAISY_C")))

